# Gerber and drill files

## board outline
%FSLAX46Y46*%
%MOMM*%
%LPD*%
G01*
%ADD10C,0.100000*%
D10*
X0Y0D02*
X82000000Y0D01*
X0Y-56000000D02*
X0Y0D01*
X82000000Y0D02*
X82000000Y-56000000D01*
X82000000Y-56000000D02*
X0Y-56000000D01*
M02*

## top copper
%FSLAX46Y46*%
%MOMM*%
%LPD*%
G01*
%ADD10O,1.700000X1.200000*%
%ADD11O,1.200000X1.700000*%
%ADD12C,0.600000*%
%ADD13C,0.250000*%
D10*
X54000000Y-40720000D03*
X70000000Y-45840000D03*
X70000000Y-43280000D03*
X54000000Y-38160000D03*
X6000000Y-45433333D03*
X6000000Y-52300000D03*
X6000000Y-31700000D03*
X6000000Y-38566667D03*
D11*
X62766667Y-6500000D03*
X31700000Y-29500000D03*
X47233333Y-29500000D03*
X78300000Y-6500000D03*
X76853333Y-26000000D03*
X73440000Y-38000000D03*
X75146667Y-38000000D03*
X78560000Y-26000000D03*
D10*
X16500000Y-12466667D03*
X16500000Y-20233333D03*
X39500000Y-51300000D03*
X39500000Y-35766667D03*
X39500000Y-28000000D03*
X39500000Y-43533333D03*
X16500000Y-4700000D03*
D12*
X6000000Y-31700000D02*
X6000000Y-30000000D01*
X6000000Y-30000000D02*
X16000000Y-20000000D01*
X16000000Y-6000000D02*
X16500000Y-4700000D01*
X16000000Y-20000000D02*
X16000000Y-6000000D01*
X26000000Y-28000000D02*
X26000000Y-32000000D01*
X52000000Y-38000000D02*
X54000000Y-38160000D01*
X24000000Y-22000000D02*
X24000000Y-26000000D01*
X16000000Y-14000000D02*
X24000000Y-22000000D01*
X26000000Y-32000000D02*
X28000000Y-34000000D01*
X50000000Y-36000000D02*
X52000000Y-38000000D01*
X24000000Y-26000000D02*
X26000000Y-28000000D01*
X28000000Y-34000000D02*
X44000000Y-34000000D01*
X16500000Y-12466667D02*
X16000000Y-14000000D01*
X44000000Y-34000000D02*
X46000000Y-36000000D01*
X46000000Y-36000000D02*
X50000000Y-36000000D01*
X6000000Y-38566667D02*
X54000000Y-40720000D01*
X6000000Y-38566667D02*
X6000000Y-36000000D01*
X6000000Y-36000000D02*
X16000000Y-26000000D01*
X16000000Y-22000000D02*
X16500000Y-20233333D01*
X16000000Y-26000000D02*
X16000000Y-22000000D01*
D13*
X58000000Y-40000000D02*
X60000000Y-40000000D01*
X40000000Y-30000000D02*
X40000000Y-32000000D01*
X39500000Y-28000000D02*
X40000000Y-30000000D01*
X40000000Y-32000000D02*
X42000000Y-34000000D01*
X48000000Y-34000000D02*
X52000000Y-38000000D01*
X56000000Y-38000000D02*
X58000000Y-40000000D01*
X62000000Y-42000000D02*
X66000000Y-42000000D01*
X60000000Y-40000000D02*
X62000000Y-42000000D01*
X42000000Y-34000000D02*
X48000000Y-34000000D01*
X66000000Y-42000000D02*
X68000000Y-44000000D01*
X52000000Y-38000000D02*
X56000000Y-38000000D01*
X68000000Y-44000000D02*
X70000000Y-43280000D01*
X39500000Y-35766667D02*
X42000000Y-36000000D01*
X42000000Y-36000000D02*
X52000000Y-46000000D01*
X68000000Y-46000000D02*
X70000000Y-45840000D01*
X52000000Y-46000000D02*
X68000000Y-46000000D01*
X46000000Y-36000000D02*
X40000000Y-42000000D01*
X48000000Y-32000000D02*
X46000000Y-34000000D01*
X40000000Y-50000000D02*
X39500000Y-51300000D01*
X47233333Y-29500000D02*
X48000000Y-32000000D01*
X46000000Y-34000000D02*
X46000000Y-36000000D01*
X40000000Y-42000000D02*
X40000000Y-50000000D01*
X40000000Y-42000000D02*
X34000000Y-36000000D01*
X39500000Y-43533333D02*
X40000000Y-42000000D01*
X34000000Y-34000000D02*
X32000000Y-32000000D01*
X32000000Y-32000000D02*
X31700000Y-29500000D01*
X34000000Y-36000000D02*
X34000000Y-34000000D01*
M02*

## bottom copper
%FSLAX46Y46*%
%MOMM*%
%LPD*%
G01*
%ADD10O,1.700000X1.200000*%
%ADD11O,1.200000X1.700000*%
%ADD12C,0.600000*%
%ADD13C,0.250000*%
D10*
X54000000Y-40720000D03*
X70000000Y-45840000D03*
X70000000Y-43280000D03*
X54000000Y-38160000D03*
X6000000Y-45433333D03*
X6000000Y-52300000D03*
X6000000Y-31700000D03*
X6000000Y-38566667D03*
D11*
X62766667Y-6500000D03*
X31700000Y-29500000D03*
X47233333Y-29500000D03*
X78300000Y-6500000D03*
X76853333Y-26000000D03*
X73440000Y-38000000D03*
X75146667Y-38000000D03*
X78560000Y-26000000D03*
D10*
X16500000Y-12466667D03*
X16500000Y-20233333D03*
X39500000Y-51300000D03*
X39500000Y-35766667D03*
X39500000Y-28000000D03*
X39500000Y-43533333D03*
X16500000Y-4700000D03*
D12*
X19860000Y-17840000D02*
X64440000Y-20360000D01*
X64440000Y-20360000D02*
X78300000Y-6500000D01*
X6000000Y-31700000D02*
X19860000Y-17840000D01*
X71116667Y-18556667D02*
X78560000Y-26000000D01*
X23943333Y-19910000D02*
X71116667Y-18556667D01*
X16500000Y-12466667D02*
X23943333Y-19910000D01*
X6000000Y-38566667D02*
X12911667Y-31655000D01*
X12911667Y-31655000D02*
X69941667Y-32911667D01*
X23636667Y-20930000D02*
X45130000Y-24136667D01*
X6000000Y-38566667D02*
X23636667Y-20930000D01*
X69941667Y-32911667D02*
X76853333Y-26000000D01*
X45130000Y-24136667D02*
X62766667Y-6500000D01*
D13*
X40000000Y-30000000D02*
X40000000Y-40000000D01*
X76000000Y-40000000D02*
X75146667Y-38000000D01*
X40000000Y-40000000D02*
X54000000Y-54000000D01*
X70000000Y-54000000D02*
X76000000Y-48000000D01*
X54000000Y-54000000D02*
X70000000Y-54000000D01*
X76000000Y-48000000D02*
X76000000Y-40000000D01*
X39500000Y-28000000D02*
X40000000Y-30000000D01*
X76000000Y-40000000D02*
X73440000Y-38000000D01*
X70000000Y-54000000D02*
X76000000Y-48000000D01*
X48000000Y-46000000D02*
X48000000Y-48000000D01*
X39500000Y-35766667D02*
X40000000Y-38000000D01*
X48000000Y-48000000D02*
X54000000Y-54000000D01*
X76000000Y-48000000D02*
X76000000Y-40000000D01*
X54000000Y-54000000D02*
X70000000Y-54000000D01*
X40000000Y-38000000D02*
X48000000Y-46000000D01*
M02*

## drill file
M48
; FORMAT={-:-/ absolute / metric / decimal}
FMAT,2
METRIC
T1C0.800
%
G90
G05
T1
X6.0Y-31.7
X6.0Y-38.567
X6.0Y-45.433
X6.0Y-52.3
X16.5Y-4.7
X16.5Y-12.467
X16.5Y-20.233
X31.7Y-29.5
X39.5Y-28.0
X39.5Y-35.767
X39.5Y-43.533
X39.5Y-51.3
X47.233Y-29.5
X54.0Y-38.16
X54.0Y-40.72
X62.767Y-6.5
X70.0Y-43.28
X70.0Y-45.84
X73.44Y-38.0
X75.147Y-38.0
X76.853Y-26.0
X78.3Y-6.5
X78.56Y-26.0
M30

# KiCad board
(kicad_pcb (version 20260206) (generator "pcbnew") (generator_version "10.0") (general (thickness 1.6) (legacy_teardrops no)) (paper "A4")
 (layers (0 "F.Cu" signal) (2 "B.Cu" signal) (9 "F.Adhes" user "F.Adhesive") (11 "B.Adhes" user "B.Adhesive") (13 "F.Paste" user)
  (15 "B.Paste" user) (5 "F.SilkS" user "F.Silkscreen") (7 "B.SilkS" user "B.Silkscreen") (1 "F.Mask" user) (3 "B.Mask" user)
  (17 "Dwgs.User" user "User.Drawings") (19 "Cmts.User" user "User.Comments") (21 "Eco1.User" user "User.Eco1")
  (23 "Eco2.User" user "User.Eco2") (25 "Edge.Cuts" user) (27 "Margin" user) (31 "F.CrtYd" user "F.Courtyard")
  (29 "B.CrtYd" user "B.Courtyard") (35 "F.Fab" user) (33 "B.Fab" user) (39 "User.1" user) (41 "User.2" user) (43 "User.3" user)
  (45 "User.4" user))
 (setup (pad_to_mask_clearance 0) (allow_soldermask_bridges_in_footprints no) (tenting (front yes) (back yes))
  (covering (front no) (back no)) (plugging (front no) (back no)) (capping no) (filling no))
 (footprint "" (layer "F.Cu") (at 62 42)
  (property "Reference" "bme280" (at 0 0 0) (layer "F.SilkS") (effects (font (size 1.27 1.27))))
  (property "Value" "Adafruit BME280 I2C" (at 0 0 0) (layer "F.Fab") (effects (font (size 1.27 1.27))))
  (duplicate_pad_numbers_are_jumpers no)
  (pad "GND" thru_hole oval (at -8 -1.28) (size 1.7 1.2) (drill 0.8) (layers "*.Cu") (remove_unused_layers no) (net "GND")
   (thermal_bridge_angle 45))
  (pad "SCL" thru_hole oval (at 8 3.84) (size 1.7 1.2) (drill 0.8) (layers "*.Cu") (remove_unused_layers no) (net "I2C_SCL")
   (thermal_bridge_angle 45))
  (pad "SDA" thru_hole oval (at 8 1.28) (size 1.7 1.2) (drill 0.8) (layers "*.Cu") (remove_unused_layers no) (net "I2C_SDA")
   (thermal_bridge_angle 45))
  (pad "VCC" thru_hole oval (at -8 -3.84) (size 1.7 1.2) (drill 0.8) (layers "*.Cu") (remove_unused_layers no) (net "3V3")
   (thermal_bridge_angle 45)))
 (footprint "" (layer "F.Cu") (at 14 42)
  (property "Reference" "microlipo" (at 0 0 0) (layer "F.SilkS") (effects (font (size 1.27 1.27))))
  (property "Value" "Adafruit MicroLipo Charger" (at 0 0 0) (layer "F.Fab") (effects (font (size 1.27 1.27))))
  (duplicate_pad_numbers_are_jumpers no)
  (pad "B+" thru_hole oval (at -8 3.433333) (size 1.7 1.2) (drill 0.8) (layers "*.Cu") (remove_unused_layers no) (thermal_bridge_angle 45))
  (pad "B-" thru_hole oval (at -8 10.3) (size 1.7 1.2) (drill 0.8) (layers "*.Cu") (remove_unused_layers no) (thermal_bridge_angle 45))
  (pad "OUT+" thru_hole oval (at -8 -10.3) (size 1.7 1.2) (drill 0.8) (layers "*.Cu") (remove_unused_layers no) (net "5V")
   (thermal_bridge_angle 45))
  (pad "OUT-" thru_hole oval (at -8 -3.433333) (size 1.7 1.2) (drill 0.8) (layers "*.Cu") (remove_unused_layers no) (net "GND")
   (thermal_bridge_angle 45)))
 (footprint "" (layer "F.Cu") (at 55 18 90)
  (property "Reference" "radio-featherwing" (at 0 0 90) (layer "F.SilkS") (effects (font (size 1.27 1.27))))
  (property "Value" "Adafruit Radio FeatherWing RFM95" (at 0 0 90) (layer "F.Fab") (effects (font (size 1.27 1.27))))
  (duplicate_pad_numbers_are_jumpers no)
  (pad "GND" thru_hole oval (at 11.5 7.766667 90) (size 1.7 1.2) (drill 0.8) (layers "*.Cu") (remove_unused_layers no) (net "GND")
   (thermal_bridge_angle 45))
  (pad "RX" thru_hole oval (at -11.5 -23.3 90) (size 1.7 1.2) (drill 0.8) (layers "*.Cu") (remove_unused_layers no) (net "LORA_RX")
   (thermal_bridge_angle 45))
  (pad "TX" thru_hole oval (at -11.5 -7.766667 90) (size 1.7 1.2) (drill 0.8) (layers "*.Cu") (remove_unused_layers no) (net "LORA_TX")
   (thermal_bridge_angle 45))
  (pad "VCC" thru_hole oval (at 11.5 23.3 90) (size 1.7 1.2) (drill 0.8) (layers "*.Cu") (remove_unused_layers no) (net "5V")
   (thermal_bridge_angle 45)))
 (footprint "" (layer "F.Cu") (at 76 32 90)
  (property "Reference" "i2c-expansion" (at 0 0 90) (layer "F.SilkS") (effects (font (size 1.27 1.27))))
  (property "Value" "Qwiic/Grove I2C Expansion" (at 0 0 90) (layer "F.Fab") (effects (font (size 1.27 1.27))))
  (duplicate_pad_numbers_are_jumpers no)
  (pad "GND" thru_hole oval (at 6 0.853333 90) (size 1.7 1.2) (drill 0.8) (layers "*.Cu") (remove_unused_layers no) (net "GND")
   (thermal_bridge_angle 45))
  (pad "SCL" thru_hole oval (at -6 -2.56 90) (size 1.7 1.2) (drill 0.8) (layers "*.Cu") (remove_unused_layers no) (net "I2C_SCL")
   (thermal_bridge_angle 45))
  (pad "SDA" thru_hole oval (at -6 -0.853333 90) (size 1.7 1.2) (drill 0.8) (layers "*.Cu") (remove_unused_layers no) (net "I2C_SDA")
   (thermal_bridge_angle 45))
  (pad "VCC" thru_hole oval (at 6 2.56 90) (size 1.7 1.2) (drill 0.8) (layers "*.Cu") (remove_unused_layers no) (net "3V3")
   (thermal_bridge_angle 45)))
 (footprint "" (layer "F.Cu") (at 28 28)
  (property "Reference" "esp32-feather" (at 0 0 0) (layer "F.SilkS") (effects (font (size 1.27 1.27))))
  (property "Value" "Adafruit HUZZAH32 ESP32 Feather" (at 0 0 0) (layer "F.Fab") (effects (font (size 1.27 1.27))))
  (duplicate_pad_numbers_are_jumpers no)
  (pad "3V3" thru_hole oval (at -11.5 -15.533333) (size 1.7 1.2) (drill 0.8) (layers "*.Cu") (remove_unused_layers no) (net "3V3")
   (thermal_bridge_angle 45))
  (pad "GND" thru_hole oval (at -11.5 -7.766667) (size 1.7 1.2) (drill 0.8) (layers "*.Cu") (remove_unused_layers no) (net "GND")
   (thermal_bridge_angle 45))
  (pad "RX" thru_hole oval (at 11.5 23.3) (size 1.7 1.2) (drill 0.8) (layers "*.Cu") (remove_unused_layers no) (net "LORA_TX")
   (thermal_bridge_angle 45))
  (pad "SCL" thru_hole oval (at 11.5 7.766667) (size 1.7 1.2) (drill 0.8) (layers "*.Cu") (remove_unused_layers no) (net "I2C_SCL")
   (thermal_bridge_angle 45))
  (pad "SDA" thru_hole oval (at 11.5 0) (size 1.7 1.2) (drill 0.8) (layers "*.Cu") (remove_unused_layers no) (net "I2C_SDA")
   (thermal_bridge_angle 45))
  (pad "TX" thru_hole oval (at 11.5 15.533333) (size 1.7 1.2) (drill 0.8) (layers "*.Cu") (remove_unused_layers no) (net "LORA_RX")
   (thermal_bridge_angle 45))
  (pad "VIN" thru_hole oval (at -11.5 -23.3) (size 1.7 1.2) (drill 0.8) (layers "*.Cu") (remove_unused_layers no) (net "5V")
   (thermal_bridge_angle 45)))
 (gr_line (start 0 0) (end 82 0) (stroke (width 0.1) (type default)) (layer "Edge.Cuts"))
 (gr_line (start 0 56) (end 0 0) (stroke (width 0.1) (type default)) (layer "Edge.Cuts"))
 (gr_line (start 82 0) (end 82 56) (stroke (width 0.1) (type default)) (layer "Edge.Cuts"))
 (gr_line (start 82 56) (end 0 56) (stroke (width 0.1) (type default)) (layer "Edge.Cuts"))
 (segment (start 6 31.7) (end 6 30) (width 0.6) (layer "F.Cu") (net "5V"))
 (segment (start 6 30) (end 16 20) (width 0.6) (layer "F.Cu") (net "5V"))
 (segment (start 16 6) (end 16.5 4.7) (width 0.6) (layer "F.Cu") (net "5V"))
 (segment (start 16 20) (end 16 6) (width 0.6) (layer "F.Cu") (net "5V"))
 (segment (start 19.86 17.84) (end 64.44 20.36) (width 0.6) (layer "B.Cu") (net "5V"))
 (segment (start 64.44 20.36) (end 78.3 6.5) (width 0.6) (layer "B.Cu") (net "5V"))
 (segment (start 6 31.7) (end 19.86 17.84) (width 0.6) (layer "B.Cu") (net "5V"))
 (segment (start 26 28) (end 26 32) (width 0.6) (layer "F.Cu") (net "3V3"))
 (segment (start 52 38) (end 54 38.16) (width 0.6) (layer "F.Cu") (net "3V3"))
 (segment (start 24 22) (end 24 26) (width 0.6) (layer "F.Cu") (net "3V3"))
 (segment (start 16 14) (end 24 22) (width 0.6) (layer "F.Cu") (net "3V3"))
 (segment (start 26 32) (end 28 34) (width 0.6) (layer "F.Cu") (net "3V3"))
 (segment (start 50 36) (end 52 38) (width 0.6) (layer "F.Cu") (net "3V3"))
 (segment (start 24 26) (end 26 28) (width 0.6) (layer "F.Cu") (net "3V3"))
 (segment (start 28 34) (end 44 34) (width 0.6) (layer "F.Cu") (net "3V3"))
 (segment (start 16.5 12.466667) (end 16 14) (width 0.6) (layer "F.Cu") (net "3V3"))
 (segment (start 44 34) (end 46 36) (width 0.6) (layer "F.Cu") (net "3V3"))
 (segment (start 46 36) (end 50 36) (width 0.6) (layer "F.Cu") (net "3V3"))
 (segment (start 71.116667 18.556667) (end 78.56 26) (width 0.6) (layer "B.Cu") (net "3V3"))
 (segment (start 23.943333 19.91) (end 71.116667 18.556667) (width 0.6) (layer "B.Cu") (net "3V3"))
 (segment (start 16.5 12.466667) (end 23.943333 19.91) (width 0.6) (layer "B.Cu") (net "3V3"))
 (segment (start 6 38.566667) (end 54 40.72) (width 0.6) (layer "F.Cu") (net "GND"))
 (segment (start 6 38.566667) (end 6 36) (width 0.6) (layer "F.Cu") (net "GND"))
 (segment (start 6 36) (end 16 26) (width 0.6) (layer "F.Cu") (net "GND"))
 (segment (start 16 22) (end 16.5 20.233333) (width 0.6) (layer "F.Cu") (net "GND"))
 (segment (start 16 26) (end 16 22) (width 0.6) (layer "F.Cu") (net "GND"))
 (segment (start 6 38.566667) (end 12.911667 31.655) (width 0.6) (layer "B.Cu") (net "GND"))
 (segment (start 12.911667 31.655) (end 69.941667 32.911667) (width 0.6) (layer "B.Cu") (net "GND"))
 (segment (start 23.636667 20.93) (end 45.13 24.136667) (width 0.6) (layer "B.Cu") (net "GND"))
 (segment (start 6 38.566667) (end 23.636667 20.93) (width 0.6) (layer "B.Cu") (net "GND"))
 (segment (start 69.941667 32.911667) (end 76.853333 26) (width 0.6) (layer "B.Cu") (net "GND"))
 (segment (start 45.13 24.136667) (end 62.766667 6.5) (width 0.6) (layer "B.Cu") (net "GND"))
 (segment (start 58 40) (end 60 40) (width 0.25) (layer "F.Cu") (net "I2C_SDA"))
 (segment (start 40 30) (end 40 32) (width 0.25) (layer "F.Cu") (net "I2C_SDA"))
 (segment (start 39.5 28) (end 40 30) (width 0.25) (layer "F.Cu") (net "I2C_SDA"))
 (segment (start 40 32) (end 42 34) (width 0.25) (layer "F.Cu") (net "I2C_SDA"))
 (segment (start 48 34) (end 52 38) (width 0.25) (layer "F.Cu") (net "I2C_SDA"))
 (segment (start 56 38) (end 58 40) (width 0.25) (layer "F.Cu") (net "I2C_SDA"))
 (segment (start 62 42) (end 66 42) (width 0.25) (layer "F.Cu") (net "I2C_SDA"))
 (segment (start 60 40) (end 62 42) (width 0.25) (layer "F.Cu") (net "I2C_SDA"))
 (segment (start 42 34) (end 48 34) (width 0.25) (layer "F.Cu") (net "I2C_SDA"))
 (segment (start 66 42) (end 68 44) (width 0.25) (layer "F.Cu") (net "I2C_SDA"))
 (segment (start 52 38) (end 56 38) (width 0.25) (layer "F.Cu") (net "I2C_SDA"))
 (segment (start 68 44) (end 70 43.28) (width 0.25) (layer "F.Cu") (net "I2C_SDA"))
 (segment (start 40 30) (end 40 40) (width 0.25) (layer "B.Cu") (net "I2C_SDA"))
 (segment (start 76 40) (end 75.146667 38) (width 0.25) (layer "B.Cu") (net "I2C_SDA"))
 (segment (start 40 40) (end 54 54) (width 0.25) (layer "B.Cu") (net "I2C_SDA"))
 (segment (start 70 54) (end 76 48) (width 0.25) (layer "B.Cu") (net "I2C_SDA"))
 (segment (start 54 54) (end 70 54) (width 0.25) (layer "B.Cu") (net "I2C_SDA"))
 (segment (start 76 48) (end 76 40) (width 0.25) (layer "B.Cu") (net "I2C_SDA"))
 (segment (start 39.5 28) (end 40 30) (width 0.25) (layer "B.Cu") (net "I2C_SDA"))
 (segment (start 39.5 35.766667) (end 42 36) (width 0.25) (layer "F.Cu") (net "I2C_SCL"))
 (segment (start 42 36) (end 52 46) (width 0.25) (layer "F.Cu") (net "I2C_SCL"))
 (segment (start 68 46) (end 70 45.84) (width 0.25) (layer "F.Cu") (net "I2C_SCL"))
 (segment (start 52 46) (end 68 46) (width 0.25) (layer "F.Cu") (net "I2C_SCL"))
 (segment (start 76 40) (end 73.44 38) (width 0.25) (layer "B.Cu") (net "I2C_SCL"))
 (segment (start 70 54) (end 76 48) (width 0.25) (layer "B.Cu") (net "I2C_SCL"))
 (segment (start 48 46) (end 48 48) (width 0.25) (layer "B.Cu") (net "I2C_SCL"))
 (segment (start 39.5 35.766667) (end 40 38) (width 0.25) (layer "B.Cu") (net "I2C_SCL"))
 (segment (start 48 48) (end 54 54) (width 0.25) (layer "B.Cu") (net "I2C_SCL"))
 (segment (start 76 48) (end 76 40) (width 0.25) (layer "B.Cu") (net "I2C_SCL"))
 (segment (start 54 54) (end 70 54) (width 0.25) (layer "B.Cu") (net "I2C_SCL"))
 (segment (start 40 38) (end 48 46) (width 0.25) (layer "B.Cu") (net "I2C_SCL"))
 (segment (start 46 36) (end 40 42) (width 0.25) (layer "F.Cu") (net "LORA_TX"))
 (segment (start 48 32) (end 46 34) (width 0.25) (layer "F.Cu") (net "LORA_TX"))
 (segment (start 40 50) (end 39.5 51.3) (width 0.25) (layer "F.Cu") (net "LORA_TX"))
 (segment (start 47.233333 29.5) (end 48 32) (width 0.25) (layer "F.Cu") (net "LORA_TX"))
 (segment (start 46 34) (end 46 36) (width 0.25) (layer "F.Cu") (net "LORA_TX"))
 (segment (start 40 42) (end 40 50) (width 0.25) (layer "F.Cu") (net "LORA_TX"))
 (segment (start 40 42) (end 34 36) (width 0.25) (layer "F.Cu") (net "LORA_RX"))
 (segment (start 39.5 43.533333) (end 40 42) (width 0.25) (layer "F.Cu") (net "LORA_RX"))
 (segment (start 34 34) (end 32 32) (width 0.25) (layer "F.Cu") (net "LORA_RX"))
 (segment (start 32 32) (end 31.7 29.5) (width 0.25) (layer "F.Cu") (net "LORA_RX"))
 (segment (start 34 36) (end 34 34) (width 0.25) (layer "F.Cu") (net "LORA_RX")))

